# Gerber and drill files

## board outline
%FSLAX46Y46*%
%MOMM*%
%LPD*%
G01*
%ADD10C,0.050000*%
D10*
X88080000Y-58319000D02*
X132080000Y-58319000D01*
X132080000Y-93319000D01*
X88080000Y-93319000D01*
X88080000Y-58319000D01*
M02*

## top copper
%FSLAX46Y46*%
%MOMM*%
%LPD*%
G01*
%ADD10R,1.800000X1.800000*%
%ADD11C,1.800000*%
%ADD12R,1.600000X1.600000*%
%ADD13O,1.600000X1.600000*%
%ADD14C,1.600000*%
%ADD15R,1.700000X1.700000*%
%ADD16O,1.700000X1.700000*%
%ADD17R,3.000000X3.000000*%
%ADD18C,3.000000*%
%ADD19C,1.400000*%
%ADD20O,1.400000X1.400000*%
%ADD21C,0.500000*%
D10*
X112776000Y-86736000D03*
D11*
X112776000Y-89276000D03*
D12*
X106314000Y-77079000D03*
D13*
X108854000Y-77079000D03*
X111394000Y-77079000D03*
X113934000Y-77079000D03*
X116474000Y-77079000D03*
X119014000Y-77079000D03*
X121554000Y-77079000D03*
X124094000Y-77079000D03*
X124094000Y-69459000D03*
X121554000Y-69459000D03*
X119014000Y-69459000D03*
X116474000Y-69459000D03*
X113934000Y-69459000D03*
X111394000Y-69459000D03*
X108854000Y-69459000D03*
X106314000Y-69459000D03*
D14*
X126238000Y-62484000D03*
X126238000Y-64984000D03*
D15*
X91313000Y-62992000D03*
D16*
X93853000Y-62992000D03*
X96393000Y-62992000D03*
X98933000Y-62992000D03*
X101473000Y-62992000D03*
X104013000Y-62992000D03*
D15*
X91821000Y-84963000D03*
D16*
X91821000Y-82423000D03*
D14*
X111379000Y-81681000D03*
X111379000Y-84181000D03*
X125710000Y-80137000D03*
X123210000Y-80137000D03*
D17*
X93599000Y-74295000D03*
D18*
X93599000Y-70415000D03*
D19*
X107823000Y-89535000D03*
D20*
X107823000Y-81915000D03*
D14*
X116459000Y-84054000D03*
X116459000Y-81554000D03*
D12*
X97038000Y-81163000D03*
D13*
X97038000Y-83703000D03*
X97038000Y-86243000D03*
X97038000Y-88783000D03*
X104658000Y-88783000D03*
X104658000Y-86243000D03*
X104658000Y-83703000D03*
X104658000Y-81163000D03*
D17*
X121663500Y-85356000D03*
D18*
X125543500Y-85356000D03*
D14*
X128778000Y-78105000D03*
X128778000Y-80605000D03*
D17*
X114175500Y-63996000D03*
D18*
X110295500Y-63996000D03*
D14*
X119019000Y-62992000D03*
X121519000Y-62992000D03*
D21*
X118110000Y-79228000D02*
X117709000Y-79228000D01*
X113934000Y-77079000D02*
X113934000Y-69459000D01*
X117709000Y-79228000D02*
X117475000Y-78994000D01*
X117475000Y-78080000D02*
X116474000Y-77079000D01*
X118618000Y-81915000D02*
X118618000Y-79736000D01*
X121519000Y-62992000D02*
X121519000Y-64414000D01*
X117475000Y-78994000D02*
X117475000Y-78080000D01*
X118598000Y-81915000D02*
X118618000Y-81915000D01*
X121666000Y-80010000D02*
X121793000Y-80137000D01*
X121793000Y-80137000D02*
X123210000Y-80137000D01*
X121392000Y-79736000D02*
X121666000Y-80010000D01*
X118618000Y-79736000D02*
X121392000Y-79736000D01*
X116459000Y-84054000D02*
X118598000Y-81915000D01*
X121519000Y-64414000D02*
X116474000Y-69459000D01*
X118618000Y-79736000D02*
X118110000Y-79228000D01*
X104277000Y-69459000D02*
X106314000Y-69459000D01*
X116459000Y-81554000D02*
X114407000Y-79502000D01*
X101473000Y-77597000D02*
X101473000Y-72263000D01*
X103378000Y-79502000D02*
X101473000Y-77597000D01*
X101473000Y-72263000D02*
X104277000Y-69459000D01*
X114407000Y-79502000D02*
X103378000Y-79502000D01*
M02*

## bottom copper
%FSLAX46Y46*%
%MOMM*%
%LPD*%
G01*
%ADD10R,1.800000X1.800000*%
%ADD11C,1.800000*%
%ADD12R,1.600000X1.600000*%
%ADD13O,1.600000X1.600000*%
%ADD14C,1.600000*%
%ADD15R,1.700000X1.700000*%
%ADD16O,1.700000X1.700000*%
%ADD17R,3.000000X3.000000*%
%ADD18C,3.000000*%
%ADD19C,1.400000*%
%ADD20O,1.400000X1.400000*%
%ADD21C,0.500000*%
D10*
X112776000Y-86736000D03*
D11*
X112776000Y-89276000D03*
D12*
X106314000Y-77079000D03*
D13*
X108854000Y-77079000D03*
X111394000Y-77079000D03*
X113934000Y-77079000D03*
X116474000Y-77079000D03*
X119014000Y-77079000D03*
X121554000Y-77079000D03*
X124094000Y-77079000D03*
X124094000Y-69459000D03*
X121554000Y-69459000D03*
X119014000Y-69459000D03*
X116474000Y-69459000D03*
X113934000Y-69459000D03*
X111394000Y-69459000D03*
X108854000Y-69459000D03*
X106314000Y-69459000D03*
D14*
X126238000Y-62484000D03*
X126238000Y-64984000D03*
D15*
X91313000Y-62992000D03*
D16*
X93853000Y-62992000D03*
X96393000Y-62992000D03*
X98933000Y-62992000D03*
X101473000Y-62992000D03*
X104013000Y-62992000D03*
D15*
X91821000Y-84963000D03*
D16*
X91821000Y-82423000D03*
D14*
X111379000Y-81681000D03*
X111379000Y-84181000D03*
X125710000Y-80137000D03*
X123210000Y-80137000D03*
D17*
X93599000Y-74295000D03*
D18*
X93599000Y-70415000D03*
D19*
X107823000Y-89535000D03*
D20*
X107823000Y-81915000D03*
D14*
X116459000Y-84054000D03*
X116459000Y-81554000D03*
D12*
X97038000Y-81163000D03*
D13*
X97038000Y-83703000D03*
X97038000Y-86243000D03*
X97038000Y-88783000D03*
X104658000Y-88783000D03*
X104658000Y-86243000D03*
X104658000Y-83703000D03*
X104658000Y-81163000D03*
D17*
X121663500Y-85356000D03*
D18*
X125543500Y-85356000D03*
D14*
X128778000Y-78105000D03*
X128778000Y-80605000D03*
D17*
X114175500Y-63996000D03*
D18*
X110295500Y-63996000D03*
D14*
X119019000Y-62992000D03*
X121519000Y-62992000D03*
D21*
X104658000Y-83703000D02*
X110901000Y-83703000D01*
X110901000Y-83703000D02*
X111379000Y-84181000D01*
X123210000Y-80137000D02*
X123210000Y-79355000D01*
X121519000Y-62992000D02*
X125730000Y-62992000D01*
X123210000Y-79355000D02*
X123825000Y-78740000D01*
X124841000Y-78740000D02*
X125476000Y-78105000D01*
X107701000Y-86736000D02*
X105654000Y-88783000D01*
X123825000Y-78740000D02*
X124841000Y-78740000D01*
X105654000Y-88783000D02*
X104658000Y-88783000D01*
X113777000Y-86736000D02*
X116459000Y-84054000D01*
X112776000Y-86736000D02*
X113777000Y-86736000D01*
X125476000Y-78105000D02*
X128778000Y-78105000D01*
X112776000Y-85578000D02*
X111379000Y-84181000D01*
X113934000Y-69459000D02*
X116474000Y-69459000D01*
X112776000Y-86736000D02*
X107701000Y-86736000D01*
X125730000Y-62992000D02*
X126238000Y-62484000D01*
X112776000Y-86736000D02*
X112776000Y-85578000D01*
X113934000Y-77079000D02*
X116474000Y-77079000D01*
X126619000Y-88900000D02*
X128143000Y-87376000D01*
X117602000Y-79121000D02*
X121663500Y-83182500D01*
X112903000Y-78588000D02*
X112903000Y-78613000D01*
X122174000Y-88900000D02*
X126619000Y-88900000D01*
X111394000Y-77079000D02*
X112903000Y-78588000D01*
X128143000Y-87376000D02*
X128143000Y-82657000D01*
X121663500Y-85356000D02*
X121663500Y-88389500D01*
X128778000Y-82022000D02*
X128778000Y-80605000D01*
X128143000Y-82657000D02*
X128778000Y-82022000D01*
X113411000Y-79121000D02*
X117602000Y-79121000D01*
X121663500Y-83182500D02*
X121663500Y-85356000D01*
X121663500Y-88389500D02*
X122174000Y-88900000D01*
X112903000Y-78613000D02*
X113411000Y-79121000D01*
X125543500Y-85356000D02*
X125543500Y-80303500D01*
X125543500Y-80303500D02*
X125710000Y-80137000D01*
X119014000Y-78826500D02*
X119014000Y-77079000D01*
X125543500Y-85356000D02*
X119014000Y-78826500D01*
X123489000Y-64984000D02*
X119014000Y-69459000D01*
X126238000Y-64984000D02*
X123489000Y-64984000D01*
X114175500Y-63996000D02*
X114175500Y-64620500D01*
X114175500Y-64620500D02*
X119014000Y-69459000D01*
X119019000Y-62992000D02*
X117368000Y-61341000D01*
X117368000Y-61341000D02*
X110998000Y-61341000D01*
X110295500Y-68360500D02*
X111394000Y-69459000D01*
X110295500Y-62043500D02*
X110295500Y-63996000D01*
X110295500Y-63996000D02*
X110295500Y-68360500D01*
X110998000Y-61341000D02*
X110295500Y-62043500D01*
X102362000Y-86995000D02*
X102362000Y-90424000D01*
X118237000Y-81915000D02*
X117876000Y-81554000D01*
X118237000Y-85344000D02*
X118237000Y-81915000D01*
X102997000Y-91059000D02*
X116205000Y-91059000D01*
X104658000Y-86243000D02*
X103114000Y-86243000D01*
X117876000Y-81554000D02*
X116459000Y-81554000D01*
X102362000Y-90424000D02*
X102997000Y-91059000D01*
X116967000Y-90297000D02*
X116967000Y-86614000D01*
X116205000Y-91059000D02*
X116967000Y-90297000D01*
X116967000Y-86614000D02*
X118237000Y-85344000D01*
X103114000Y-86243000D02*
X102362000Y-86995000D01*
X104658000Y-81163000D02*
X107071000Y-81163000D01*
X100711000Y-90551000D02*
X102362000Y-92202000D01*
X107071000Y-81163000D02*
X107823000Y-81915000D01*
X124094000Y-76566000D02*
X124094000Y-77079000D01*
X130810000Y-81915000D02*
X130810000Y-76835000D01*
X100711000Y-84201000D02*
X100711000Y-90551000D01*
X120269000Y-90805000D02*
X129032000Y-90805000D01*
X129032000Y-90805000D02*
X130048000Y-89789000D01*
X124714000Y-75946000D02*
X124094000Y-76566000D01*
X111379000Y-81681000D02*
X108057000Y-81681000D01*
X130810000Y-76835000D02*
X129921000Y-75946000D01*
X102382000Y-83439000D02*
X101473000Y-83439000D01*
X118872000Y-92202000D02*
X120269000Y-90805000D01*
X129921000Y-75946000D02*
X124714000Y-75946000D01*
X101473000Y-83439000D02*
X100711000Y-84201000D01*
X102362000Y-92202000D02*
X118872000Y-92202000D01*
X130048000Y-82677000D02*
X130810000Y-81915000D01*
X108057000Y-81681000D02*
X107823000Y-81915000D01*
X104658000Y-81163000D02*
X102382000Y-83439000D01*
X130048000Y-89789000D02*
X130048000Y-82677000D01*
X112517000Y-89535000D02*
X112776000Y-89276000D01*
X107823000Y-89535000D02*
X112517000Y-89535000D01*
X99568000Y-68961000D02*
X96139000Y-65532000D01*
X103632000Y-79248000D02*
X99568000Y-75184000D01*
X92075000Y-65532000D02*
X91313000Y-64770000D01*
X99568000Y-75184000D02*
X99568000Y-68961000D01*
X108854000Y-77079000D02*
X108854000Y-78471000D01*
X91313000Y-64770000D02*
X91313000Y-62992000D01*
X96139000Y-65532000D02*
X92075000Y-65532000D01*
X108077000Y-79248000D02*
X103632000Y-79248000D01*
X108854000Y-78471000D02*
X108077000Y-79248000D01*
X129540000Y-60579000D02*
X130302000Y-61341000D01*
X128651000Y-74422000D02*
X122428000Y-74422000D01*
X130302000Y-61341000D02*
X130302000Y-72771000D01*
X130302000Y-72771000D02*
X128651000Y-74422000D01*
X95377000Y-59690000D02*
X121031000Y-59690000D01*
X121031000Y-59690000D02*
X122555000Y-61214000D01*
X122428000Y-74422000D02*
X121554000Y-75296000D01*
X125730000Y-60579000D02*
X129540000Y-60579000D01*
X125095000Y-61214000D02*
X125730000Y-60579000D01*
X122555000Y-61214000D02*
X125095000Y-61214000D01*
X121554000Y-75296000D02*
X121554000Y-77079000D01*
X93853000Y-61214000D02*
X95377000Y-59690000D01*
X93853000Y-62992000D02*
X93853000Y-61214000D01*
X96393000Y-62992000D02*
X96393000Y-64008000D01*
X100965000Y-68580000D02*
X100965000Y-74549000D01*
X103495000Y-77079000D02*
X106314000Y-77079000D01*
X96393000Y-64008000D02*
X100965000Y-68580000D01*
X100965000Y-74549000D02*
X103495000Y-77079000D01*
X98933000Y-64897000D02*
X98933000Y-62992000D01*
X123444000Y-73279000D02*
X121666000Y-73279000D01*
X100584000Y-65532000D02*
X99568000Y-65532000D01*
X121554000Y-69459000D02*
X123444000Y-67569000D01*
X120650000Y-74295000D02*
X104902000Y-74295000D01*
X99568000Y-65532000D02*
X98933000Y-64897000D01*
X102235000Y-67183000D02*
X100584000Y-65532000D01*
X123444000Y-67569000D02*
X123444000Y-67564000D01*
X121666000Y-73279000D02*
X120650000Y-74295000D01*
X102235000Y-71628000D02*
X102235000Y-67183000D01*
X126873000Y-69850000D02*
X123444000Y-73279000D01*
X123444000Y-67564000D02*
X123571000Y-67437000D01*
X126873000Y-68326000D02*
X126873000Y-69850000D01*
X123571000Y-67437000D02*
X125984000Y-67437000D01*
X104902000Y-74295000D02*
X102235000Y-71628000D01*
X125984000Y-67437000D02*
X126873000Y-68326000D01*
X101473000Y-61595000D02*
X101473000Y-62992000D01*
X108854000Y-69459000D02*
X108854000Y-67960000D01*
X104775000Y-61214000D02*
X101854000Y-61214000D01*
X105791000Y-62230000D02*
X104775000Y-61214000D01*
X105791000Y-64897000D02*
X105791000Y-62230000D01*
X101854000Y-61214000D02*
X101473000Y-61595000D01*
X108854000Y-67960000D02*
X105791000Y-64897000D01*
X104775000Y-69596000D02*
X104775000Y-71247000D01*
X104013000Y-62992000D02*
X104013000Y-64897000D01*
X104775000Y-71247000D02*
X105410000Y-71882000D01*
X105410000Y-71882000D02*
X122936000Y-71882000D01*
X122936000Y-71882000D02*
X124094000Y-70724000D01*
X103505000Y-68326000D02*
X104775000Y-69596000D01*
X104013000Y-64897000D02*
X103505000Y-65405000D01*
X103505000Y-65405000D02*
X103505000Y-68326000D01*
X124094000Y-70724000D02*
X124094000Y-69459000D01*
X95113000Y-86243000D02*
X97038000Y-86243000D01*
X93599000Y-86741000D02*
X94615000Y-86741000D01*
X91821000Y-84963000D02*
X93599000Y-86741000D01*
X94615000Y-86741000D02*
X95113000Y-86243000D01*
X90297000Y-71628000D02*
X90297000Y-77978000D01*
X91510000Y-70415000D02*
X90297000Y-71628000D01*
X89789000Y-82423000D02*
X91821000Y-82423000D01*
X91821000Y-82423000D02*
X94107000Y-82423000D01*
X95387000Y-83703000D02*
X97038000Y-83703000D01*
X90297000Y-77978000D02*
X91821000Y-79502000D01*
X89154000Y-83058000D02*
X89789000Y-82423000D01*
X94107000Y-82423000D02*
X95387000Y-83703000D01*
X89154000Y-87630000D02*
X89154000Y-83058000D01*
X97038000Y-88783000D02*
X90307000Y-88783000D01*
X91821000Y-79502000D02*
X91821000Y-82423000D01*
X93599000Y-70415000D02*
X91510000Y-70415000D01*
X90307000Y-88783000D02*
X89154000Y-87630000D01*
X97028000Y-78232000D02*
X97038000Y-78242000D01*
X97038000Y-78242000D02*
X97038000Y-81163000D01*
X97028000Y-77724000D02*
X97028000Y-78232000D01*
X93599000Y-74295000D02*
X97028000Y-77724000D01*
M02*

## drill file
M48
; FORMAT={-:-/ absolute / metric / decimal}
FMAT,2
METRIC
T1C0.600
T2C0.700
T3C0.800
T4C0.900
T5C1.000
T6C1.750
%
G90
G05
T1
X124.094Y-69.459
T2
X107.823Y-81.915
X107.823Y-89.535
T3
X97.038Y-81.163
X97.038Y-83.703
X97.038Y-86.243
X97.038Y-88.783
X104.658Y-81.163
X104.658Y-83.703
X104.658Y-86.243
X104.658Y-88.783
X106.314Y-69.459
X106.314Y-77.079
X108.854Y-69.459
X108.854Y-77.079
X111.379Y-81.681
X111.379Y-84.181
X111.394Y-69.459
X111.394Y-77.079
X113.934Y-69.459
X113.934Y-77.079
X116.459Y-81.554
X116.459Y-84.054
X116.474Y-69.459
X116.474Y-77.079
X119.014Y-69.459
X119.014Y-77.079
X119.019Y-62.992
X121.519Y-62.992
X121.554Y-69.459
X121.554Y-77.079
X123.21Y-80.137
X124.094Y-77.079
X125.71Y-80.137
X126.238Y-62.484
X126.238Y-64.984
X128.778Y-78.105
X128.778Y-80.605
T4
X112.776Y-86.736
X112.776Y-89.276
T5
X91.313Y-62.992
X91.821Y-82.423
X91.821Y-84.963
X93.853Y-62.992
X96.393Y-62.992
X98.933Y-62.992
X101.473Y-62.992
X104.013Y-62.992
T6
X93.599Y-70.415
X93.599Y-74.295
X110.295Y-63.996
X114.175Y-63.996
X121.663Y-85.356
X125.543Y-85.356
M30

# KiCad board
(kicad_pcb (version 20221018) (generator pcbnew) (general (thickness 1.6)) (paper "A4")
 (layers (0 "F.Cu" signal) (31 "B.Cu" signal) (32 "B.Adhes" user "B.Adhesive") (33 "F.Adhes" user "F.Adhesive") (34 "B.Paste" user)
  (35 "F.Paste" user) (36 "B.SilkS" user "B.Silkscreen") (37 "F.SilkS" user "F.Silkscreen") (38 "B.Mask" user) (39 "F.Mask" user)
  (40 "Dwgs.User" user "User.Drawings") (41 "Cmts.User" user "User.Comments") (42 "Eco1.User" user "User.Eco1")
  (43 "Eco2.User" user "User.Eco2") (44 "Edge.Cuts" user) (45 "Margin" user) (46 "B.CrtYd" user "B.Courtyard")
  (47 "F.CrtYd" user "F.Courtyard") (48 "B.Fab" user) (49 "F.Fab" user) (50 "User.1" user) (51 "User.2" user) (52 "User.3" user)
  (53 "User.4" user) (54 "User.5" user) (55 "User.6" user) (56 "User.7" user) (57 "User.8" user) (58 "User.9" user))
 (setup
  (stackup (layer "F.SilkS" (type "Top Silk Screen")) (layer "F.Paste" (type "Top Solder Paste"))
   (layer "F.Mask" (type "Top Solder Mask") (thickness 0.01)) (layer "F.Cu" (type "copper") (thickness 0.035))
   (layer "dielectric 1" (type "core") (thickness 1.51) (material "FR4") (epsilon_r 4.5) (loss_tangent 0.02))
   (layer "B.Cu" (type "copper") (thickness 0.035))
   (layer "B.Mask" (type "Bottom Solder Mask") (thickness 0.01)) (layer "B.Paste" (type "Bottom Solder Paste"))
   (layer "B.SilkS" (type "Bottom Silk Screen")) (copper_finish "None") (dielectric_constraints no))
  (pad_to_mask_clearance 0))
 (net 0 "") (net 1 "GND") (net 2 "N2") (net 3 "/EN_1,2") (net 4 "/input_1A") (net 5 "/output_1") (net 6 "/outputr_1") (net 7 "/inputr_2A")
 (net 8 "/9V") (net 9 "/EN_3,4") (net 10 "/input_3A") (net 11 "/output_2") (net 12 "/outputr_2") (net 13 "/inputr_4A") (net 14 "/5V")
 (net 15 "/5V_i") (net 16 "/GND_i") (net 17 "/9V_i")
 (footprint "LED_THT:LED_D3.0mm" (layer "F.Cu") (at 112.776 86.736 -90)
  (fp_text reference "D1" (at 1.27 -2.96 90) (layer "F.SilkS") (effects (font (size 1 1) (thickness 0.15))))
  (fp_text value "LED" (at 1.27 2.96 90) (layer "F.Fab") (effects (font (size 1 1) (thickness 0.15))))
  (pad "1" thru_hole rect (at 0 0 270) (size 1.8 1.8) (drill 0.9) (layers "*.Cu" "*.Mask") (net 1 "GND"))
  (pad "2" thru_hole circle (at 2.54 0 270) (size 1.8 1.8) (drill 0.9) (layers "*.Cu" "*.Mask") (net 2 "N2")))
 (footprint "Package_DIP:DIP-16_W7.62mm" (layer "F.Cu") (at 106.314 77.079 90)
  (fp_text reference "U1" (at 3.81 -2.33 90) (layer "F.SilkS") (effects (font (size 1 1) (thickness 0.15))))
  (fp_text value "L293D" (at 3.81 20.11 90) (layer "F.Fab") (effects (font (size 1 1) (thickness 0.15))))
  (pad "1" thru_hole rect (at 0 0 90) (size 1.6 1.6) (drill 0.8) (layers "*.Cu" "*.Mask") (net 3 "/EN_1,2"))
  (pad "2" thru_hole oval (at 0 2.54 90) (size 1.6 1.6) (drill 0.8) (layers "*.Cu" "*.Mask") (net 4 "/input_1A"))
  (pad "3" thru_hole oval (at 0 5.08 90) (size 1.6 1.6) (drill 0.8) (layers "*.Cu" "*.Mask") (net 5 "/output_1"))
  (pad "4" thru_hole oval (at 0 7.62 90) (size 1.6 1.6) (drill 0.8) (layers "*.Cu" "*.Mask") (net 1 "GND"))
  (pad "5" thru_hole oval (at 0 10.16 90) (size 1.6 1.6) (drill 0.8) (layers "*.Cu" "*.Mask") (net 1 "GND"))
  (pad "6" thru_hole oval (at 0 12.7 90) (size 1.6 1.6) (drill 0.8) (layers "*.Cu" "*.Mask") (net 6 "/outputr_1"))
  (pad "7" thru_hole oval (at 0 15.24 90) (size 1.6 1.6) (drill 0.8) (layers "*.Cu" "*.Mask") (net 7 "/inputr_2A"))
  (pad "8" thru_hole oval (at 0 17.78 90) (size 1.6 1.6) (drill 0.8) (layers "*.Cu" "*.Mask") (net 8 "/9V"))
  (pad "9" thru_hole oval (at 7.62 17.78 90) (size 1.6 1.6) (drill 0.6) (layers "*.Cu" "*.Mask") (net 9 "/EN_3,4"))
  (pad "10" thru_hole oval (at 7.62 15.24 90) (size 1.6 1.6) (drill 0.8) (layers "*.Cu" "*.Mask") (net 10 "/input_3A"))
  (pad "11" thru_hole oval (at 7.62 12.7 90) (size 1.6 1.6) (drill 0.8) (layers "*.Cu" "*.Mask") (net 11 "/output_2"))
  (pad "12" thru_hole oval (at 7.62 10.16 90) (size 1.6 1.6) (drill 0.8) (layers "*.Cu" "*.Mask") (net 1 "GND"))
  (pad "13" thru_hole oval (at 7.62 7.62 90) (size 1.6 1.6) (drill 0.8) (layers "*.Cu" "*.Mask") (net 1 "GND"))
  (pad "14" thru_hole oval (at 7.62 5.08 90) (size 1.6 1.6) (drill 0.8) (layers "*.Cu" "*.Mask") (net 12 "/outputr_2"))
  (pad "15" thru_hole oval (at 7.62 2.54 90) (size 1.6 1.6) (drill 0.8) (layers "*.Cu" "*.Mask") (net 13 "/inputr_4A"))
  (pad "16" thru_hole oval (at 7.62 0 90) (size 1.6 1.6) (drill 0.8) (layers "*.Cu" "*.Mask") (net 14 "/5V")))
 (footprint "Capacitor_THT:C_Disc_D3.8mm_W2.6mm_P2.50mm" (layer "F.Cu") (at 126.238 62.484 -90)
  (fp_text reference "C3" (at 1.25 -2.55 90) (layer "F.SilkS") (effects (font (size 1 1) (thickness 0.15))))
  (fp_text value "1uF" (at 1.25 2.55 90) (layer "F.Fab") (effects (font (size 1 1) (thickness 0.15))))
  (pad "1" thru_hole circle (at 0 0 270) (size 1.6 1.6) (drill 0.8) (layers "*.Cu" "*.Mask") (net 1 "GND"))
  (pad "2" thru_hole circle (at 2.5 0 270) (size 1.6 1.6) (drill 0.8) (layers "*.Cu" "*.Mask") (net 11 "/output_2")))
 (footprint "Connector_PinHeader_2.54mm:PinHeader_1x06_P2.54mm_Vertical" (layer "F.Cu") (at 91.313 62.992 90)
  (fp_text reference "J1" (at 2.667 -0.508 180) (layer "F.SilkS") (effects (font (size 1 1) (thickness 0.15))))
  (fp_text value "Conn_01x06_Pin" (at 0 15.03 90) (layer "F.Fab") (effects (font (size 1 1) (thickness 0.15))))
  (pad "1" thru_hole rect (at 0 0 90) (size 1.7 1.7) (drill 1) (layers "*.Cu" "*.Mask") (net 4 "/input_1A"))
  (pad "2" thru_hole oval (at 0 2.54 90) (size 1.7 1.7) (drill 1) (layers "*.Cu" "*.Mask") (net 7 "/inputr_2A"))
  (pad "3" thru_hole oval (at 0 5.08 90) (size 1.7 1.7) (drill 1) (layers "*.Cu" "*.Mask") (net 3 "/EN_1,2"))
  (pad "4" thru_hole oval (at 0 7.62 90) (size 1.7 1.7) (drill 1) (layers "*.Cu" "*.Mask") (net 10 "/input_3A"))
  (pad "5" thru_hole oval (at 0 10.16 90) (size 1.7 1.7) (drill 1) (layers "*.Cu" "*.Mask") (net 13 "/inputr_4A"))
  (pad "6" thru_hole oval (at 0 12.7 90) (size 1.7 1.7) (drill 1) (layers "*.Cu" "*.Mask") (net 9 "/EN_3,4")))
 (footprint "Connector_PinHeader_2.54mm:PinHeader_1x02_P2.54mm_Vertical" (layer "F.Cu") (at 91.821 84.963 180)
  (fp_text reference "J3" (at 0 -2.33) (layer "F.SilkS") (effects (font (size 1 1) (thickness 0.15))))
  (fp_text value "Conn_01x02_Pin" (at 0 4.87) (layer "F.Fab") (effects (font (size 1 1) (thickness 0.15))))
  (pad "1" thru_hole rect (at 0 0 180) (size 1.7 1.7) (drill 1) (layers "*.Cu" "*.Mask") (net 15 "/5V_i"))
  (pad "2" thru_hole oval (at 0 2.54 180) (size 1.7 1.7) (drill 1) (layers "*.Cu" "*.Mask") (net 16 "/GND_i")))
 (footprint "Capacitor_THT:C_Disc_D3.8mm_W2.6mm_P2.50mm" (layer "F.Cu") (at 111.379 81.681 -90)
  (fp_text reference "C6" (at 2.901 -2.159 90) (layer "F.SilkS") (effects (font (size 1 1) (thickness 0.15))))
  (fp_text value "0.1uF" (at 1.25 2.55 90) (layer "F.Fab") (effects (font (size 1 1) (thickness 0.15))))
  (pad "1" thru_hole circle (at 0 0 270) (size 1.6 1.6) (drill 0.8) (layers "*.Cu" "*.Mask") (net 8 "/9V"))
  (pad "2" thru_hole circle (at 2.5 0 270) (size 1.6 1.6) (drill 0.8) (layers "*.Cu" "*.Mask") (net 1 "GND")))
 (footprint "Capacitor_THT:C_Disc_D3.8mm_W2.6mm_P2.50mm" (layer "F.Cu") (at 125.71 80.137 180)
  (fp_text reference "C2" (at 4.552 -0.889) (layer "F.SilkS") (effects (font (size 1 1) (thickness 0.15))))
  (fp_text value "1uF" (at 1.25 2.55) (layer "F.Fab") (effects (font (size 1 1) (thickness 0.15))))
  (pad "1" thru_hole circle (at 0 0 180) (size 1.6 1.6) (drill 0.8) (layers "*.Cu" "*.Mask") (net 6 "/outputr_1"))
  (pad "2" thru_hole circle (at 2.5 0 180) (size 1.6 1.6) (drill 0.8) (layers "*.Cu" "*.Mask") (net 1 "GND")))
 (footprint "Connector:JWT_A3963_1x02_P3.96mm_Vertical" (layer "F.Cu") (at 93.599 74.295 90)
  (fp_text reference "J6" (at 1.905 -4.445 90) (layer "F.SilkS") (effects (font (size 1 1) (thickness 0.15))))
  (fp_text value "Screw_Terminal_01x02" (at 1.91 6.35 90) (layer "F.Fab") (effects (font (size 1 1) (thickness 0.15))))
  (pad "1" thru_hole rect (at 0 0 90) (size 3 3) (drill 1.75) (layers "*.Cu" "*.Mask") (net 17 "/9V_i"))
  (pad "2" thru_hole circle (at 3.88 0 90) (size 3 3) (drill 1.75) (layers "*.Cu" "*.Mask") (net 16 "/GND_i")))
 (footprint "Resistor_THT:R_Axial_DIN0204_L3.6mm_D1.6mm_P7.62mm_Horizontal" (layer "F.Cu") (at 107.823 89.535 90)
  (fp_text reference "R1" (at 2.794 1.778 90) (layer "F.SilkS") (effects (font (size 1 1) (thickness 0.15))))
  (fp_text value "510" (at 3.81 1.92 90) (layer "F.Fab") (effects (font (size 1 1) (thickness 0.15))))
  (pad "1" thru_hole circle (at 0 0 90) (size 1.4 1.4) (drill 0.7) (layers "*.Cu" "*.Mask") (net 2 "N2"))
  (pad "2" thru_hole oval (at 7.62 0 90) (size 1.4 1.4) (drill 0.7) (layers "*.Cu" "*.Mask") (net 8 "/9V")))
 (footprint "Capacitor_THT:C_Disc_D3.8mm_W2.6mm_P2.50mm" (layer "F.Cu") (at 116.459 84.054 90)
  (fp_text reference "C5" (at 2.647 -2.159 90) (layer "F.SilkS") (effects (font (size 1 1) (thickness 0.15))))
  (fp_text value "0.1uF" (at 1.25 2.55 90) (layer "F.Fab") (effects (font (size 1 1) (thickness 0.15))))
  (pad "1" thru_hole circle (at 0 0 90) (size 1.6 1.6) (drill 0.8) (layers "*.Cu" "*.Mask") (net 1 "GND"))
  (pad "2" thru_hole circle (at 2.5 0 90) (size 1.6 1.6) (drill 0.8) (layers "*.Cu" "*.Mask") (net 14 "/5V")))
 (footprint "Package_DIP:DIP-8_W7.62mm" (layer "F.Cu") (at 97.038 81.163)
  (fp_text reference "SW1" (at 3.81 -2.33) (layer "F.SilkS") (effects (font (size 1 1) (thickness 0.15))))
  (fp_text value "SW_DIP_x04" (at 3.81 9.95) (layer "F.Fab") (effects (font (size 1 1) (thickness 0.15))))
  (pad "1" thru_hole rect (at 0 0) (size 1.6 1.6) (drill 0.8) (layers "*.Cu" "*.Mask") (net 17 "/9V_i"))
  (pad "2" thru_hole oval (at 0 2.54) (size 1.6 1.6) (drill 0.8) (layers "*.Cu" "*.Mask") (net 16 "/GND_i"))
  (pad "3" thru_hole oval (at 0 5.08) (size 1.6 1.6) (drill 0.8) (layers "*.Cu" "*.Mask") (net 15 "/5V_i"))
  (pad "4" thru_hole oval (at 0 7.62) (size 1.6 1.6) (drill 0.8) (layers "*.Cu" "*.Mask") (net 16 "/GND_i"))
  (pad "5" thru_hole oval (at 7.62 7.62) (size 1.6 1.6) (drill 0.8) (layers "*.Cu" "*.Mask") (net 1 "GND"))
  (pad "6" thru_hole oval (at 7.62 5.08) (size 1.6 1.6) (drill 0.8) (layers "*.Cu" "*.Mask") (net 14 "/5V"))
  (pad "7" thru_hole oval (at 7.62 2.54) (size 1.6 1.6) (drill 0.8) (layers "*.Cu" "*.Mask") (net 1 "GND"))
  (pad "8" thru_hole oval (at 7.62 0) (size 1.6 1.6) (drill 0.8) (layers "*.Cu" "*.Mask") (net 8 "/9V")))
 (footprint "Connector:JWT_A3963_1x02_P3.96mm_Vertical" (layer "F.Cu") (at 121.6635 85.356)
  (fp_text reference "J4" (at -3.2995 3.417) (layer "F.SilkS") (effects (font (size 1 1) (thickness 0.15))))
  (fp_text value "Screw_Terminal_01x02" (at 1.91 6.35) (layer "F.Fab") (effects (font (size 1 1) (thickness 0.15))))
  (pad "1" thru_hole rect (at 0 0) (size 3 3) (drill 1.75) (layers "*.Cu" "*.Mask") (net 5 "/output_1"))
  (pad "2" thru_hole circle (at 3.88 0) (size 3 3) (drill 1.75) (layers "*.Cu" "*.Mask") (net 6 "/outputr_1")))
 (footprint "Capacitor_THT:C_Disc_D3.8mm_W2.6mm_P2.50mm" (layer "F.Cu") (at 128.778 78.105 -90)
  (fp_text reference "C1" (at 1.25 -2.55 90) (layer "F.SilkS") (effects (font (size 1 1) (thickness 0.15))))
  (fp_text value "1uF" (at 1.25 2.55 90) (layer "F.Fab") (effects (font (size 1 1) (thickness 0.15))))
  (pad "1" thru_hole circle (at 0 0 270) (size 1.6 1.6) (drill 0.8) (layers "*.Cu" "*.Mask") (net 1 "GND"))
  (pad "2" thru_hole circle (at 2.5 0 270) (size 1.6 1.6) (drill 0.8) (layers "*.Cu" "*.Mask") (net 5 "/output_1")))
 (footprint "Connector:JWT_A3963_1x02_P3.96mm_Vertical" (layer "F.Cu") (at 114.1755 63.996 180)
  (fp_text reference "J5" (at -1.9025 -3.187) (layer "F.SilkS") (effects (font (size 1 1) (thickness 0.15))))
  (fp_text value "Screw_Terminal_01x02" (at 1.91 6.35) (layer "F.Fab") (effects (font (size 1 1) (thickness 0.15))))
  (pad "1" thru_hole rect (at 0 0 180) (size 3 3) (drill 1.75) (layers "*.Cu" "*.Mask") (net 11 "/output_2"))
  (pad "2" thru_hole circle (at 3.88 0 180) (size 3 3) (drill 1.75) (layers "*.Cu" "*.Mask") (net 12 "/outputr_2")))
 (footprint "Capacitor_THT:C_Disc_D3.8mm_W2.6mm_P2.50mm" (layer "F.Cu") (at 119.019 62.992)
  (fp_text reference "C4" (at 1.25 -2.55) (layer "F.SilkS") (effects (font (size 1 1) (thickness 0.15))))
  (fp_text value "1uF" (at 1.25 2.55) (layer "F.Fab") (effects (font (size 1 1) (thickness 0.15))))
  (pad "1" thru_hole circle (at 0 0) (size 1.6 1.6) (drill 0.8) (layers "*.Cu" "*.Mask") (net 12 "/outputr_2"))
  (pad "2" thru_hole circle (at 2.5 0) (size 1.6 1.6) (drill 0.8) (layers "*.Cu" "*.Mask") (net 1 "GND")))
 (gr_rect (start 88.08 58.319) (end 132.08 93.319) (stroke (width 0.05) (type default)) (fill none) (layer "Edge.Cuts"))
 (segment (start 118.11 79.228) (end 117.709 79.228) (width 0.5) (layer "F.Cu") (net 1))
 (segment (start 113.934 77.079) (end 113.934 69.459) (width 0.5) (layer "F.Cu") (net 1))
 (segment (start 117.709 79.228) (end 117.475 78.994) (width 0.5) (layer "F.Cu") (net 1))
 (segment (start 117.475 78.08) (end 116.474 77.079) (width 0.5) (layer "F.Cu") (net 1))
 (segment (start 118.618 81.915) (end 118.618 79.736) (width 0.5) (layer "F.Cu") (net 1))
 (segment (start 121.519 62.992) (end 121.519 64.414) (width 0.5) (layer "F.Cu") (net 1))
 (segment (start 117.475 78.994) (end 117.475 78.08) (width 0.5) (layer "F.Cu") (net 1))
 (segment (start 118.598 81.915) (end 118.618 81.915) (width 0.5) (layer "F.Cu") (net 1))
 (segment (start 121.666 80.01) (end 121.793 80.137) (width 0.5) (layer "F.Cu") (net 1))
 (segment (start 121.793 80.137) (end 123.21 80.137) (width 0.5) (layer "F.Cu") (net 1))
 (segment (start 121.392 79.736) (end 121.666 80.01) (width 0.5) (layer "F.Cu") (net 1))
 (segment (start 118.618 79.736) (end 121.392 79.736) (width 0.5) (layer "F.Cu") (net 1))
 (segment (start 116.459 84.054) (end 118.598 81.915) (width 0.5) (layer "F.Cu") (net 1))
 (segment (start 121.519 64.414) (end 116.474 69.459) (width 0.5) (layer "F.Cu") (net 1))
 (segment (start 118.618 79.736) (end 118.11 79.228) (width 0.5) (layer "F.Cu") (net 1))
 (segment (start 104.658 83.703) (end 110.901 83.703) (width 0.5) (layer "B.Cu") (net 1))
 (segment (start 110.901 83.703) (end 111.379 84.181) (width 0.5) (layer "B.Cu") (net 1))
 (segment (start 123.21 80.137) (end 123.21 79.355) (width 0.5) (layer "B.Cu") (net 1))
 (segment (start 121.519 62.992) (end 125.73 62.992) (width 0.5) (layer "B.Cu") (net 1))
 (segment (start 123.21 79.355) (end 123.825 78.74) (width 0.5) (layer "B.Cu") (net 1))
 (segment (start 124.841 78.74) (end 125.476 78.105) (width 0.5) (layer "B.Cu") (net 1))
 (segment (start 107.701 86.736) (end 105.654 88.783) (width 0.5) (layer "B.Cu") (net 1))
 (segment (start 123.825 78.74) (end 124.841 78.74) (width 0.5) (layer "B.Cu") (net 1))
 (segment (start 105.654 88.783) (end 104.658 88.783) (width 0.5) (layer "B.Cu") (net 1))
 (segment (start 113.777 86.736) (end 116.459 84.054) (width 0.5) (layer "B.Cu") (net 1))
 (segment (start 112.776 86.736) (end 113.777 86.736) (width 0.5) (layer "B.Cu") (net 1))
 (segment (start 125.476 78.105) (end 128.778 78.105) (width 0.5) (layer "B.Cu") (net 1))
 (segment (start 112.776 85.578) (end 111.379 84.181) (width 0.5) (layer "B.Cu") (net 1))
 (segment (start 113.934 69.459) (end 116.474 69.459) (width 0.5) (layer "B.Cu") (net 1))
 (segment (start 112.776 86.736) (end 107.701 86.736) (width 0.5) (layer "B.Cu") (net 1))
 (segment (start 125.73 62.992) (end 126.238 62.484) (width 0.5) (layer "B.Cu") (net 1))
 (segment (start 112.776 86.736) (end 112.776 85.578) (width 0.5) (layer "B.Cu") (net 1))
 (segment (start 113.934 77.079) (end 116.474 77.079) (width 0.5) (layer "B.Cu") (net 1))
 (segment (start 126.619 88.9) (end 128.143 87.376) (width 0.5) (layer "B.Cu") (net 5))
 (segment (start 117.602 79.121) (end 121.6635 83.1825) (width 0.5) (layer "B.Cu") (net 5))
 (segment (start 112.903 78.588) (end 112.903 78.613) (width 0.5) (layer "B.Cu") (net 5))
 (segment (start 122.174 88.9) (end 126.619 88.9) (width 0.5) (layer "B.Cu") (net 5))
 (segment (start 111.394 77.079) (end 112.903 78.588) (width 0.5) (layer "B.Cu") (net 5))
 (segment (start 128.143 87.376) (end 128.143 82.657) (width 0.5) (layer "B.Cu") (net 5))
 (segment (start 121.6635 85.356) (end 121.6635 88.3895) (width 0.5) (layer "B.Cu") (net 5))
 (segment (start 128.778 82.022) (end 128.778 80.605) (width 0.5) (layer "B.Cu") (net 5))
 (segment (start 128.143 82.657) (end 128.778 82.022) (width 0.5) (layer "B.Cu") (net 5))
 (segment (start 113.411 79.121) (end 117.602 79.121) (width 0.5) (layer "B.Cu") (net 5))
 (segment (start 121.6635 83.1825) (end 121.6635 85.356) (width 0.5) (layer "B.Cu") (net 5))
 (segment (start 121.6635 88.3895) (end 122.174 88.9) (width 0.5) (layer "B.Cu") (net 5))
 (segment (start 112.903 78.613) (end 113.411 79.121) (width 0.5) (layer "B.Cu") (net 5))
 (segment (start 125.5435 85.356) (end 125.5435 80.3035) (width 0.5) (layer "B.Cu") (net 6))
 (segment (start 125.5435 80.3035) (end 125.71 80.137) (width 0.5) (layer "B.Cu") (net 6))
 (segment (start 119.014 78.8265) (end 119.014 77.079) (width 0.5) (layer "B.Cu") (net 6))
 (segment (start 125.5435 85.356) (end 119.014 78.8265) (width 0.5) (layer "B.Cu") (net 6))
 (segment (start 123.489 64.984) (end 119.014 69.459) (width 0.5) (layer "B.Cu") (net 11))
 (segment (start 126.238 64.984) (end 123.489 64.984) (width 0.5) (layer "B.Cu") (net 11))
 (segment (start 114.1755 63.996) (end 114.1755 64.6205) (width 0.5) (layer "B.Cu") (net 11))
 (segment (start 114.1755 64.6205) (end 119.014 69.459) (width 0.5) (layer "B.Cu") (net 11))
 (segment (start 119.019 62.992) (end 117.368 61.341) (width 0.5) (layer "B.Cu") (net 12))
 (segment (start 117.368 61.341) (end 110.998 61.341) (width 0.5) (layer "B.Cu") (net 12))
 (segment (start 110.2955 68.3605) (end 111.394 69.459) (width 0.5) (layer "B.Cu") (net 12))
 (segment (start 110.2955 62.0435) (end 110.2955 63.996) (width 0.5) (layer "B.Cu") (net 12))
 (segment (start 110.2955 63.996) (end 110.2955 68.3605) (width 0.5) (layer "B.Cu") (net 12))
 (segment (start 110.998 61.341) (end 110.2955 62.0435) (width 0.5) (layer "B.Cu") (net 12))
 (segment (start 104.277 69.459) (end 106.314 69.459) (width 0.5) (layer "F.Cu") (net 14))
 (segment (start 116.459 81.554) (end 114.407 79.502) (width 0.5) (layer "F.Cu") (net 14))
 (segment (start 101.473 77.597) (end 101.473 72.263) (width 0.5) (layer "F.Cu") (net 14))
 (segment (start 103.378 79.502) (end 101.473 77.597) (width 0.5) (layer "F.Cu") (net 14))
 (segment (start 101.473 72.263) (end 104.277 69.459) (width 0.5) (layer "F.Cu") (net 14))
 (segment (start 114.407 79.502) (end 103.378 79.502) (width 0.5) (layer "F.Cu") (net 14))
 (segment (start 102.362 86.995) (end 102.362 90.424) (width 0.5) (layer "B.Cu") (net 14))
 (segment (start 118.237 81.915) (end 117.876 81.554) (width 0.5) (layer "B.Cu") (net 14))
 (segment (start 118.237 85.344) (end 118.237 81.915) (width 0.5) (layer "B.Cu") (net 14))
 (segment (start 102.997 91.059) (end 116.205 91.059) (width 0.5) (layer "B.Cu") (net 14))
 (segment (start 104.658 86.243) (end 103.114 86.243) (width 0.5) (layer "B.Cu") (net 14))
 (segment (start 117.876 81.554) (end 116.459 81.554) (width 0.5) (layer "B.Cu") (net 14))
 (segment (start 102.362 90.424) (end 102.997 91.059) (width 0.5) (layer "B.Cu") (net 14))
 (segment (start 116.967 90.297) (end 116.967 86.614) (width 0.5) (layer "B.Cu") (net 14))
 (segment (start 116.205 91.059) (end 116.967 90.297) (width 0.5) (layer "B.Cu") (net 14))
 (segment (start 116.967 86.614) (end 118.237 85.344) (width 0.5) (layer "B.Cu") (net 14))
 (segment (start 103.114 86.243) (end 102.362 86.995) (width 0.5) (layer "B.Cu") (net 14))
 (segment (start 104.658 81.163) (end 107.071 81.163) (width 0.5) (layer "B.Cu") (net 8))
 (segment (start 100.711 90.551) (end 102.362 92.202) (width 0.5) (layer "B.Cu") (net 8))
 (segment (start 107.071 81.163) (end 107.823 81.915) (width 0.5) (layer "B.Cu") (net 8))
 (segment (start 124.094 76.566) (end 124.094 77.079) (width 0.5) (layer "B.Cu") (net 8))
 (segment (start 130.81 81.915) (end 130.81 76.835) (width 0.5) (layer "B.Cu") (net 8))
 (segment (start 100.711 84.201) (end 100.711 90.551) (width 0.5) (layer "B.Cu") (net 8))
 (segment (start 120.269 90.805) (end 129.032 90.805) (width 0.5) (layer "B.Cu") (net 8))
 (segment (start 129.032 90.805) (end 130.048 89.789) (width 0.5) (layer "B.Cu") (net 8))
 (segment (start 124.714 75.946) (end 124.094 76.566) (width 0.5) (layer "B.Cu") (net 8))
 (segment (start 111.379 81.681) (end 108.057 81.681) (width 0.5) (layer "B.Cu") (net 8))
 (segment (start 130.81 76.835) (end 129.921 75.946) (width 0.5) (layer "B.Cu") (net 8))
 (segment (start 102.382 83.439) (end 101.473 83.439) (width 0.5) (layer "B.Cu") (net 8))
 (segment (start 118.872 92.202) (end 120.269 90.805) (width 0.5) (layer "B.Cu") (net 8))
 (segment (start 129.921 75.946) (end 124.714 75.946) (width 0.5) (layer "B.Cu") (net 8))
 (segment (start 101.473 83.439) (end 100.711 84.201) (width 0.5) (layer "B.Cu") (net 8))
 (segment (start 102.362 92.202) (end 118.872 92.202) (width 0.5) (layer "B.Cu") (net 8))
 (segment (start 130.048 82.677) (end 130.81 81.915) (width 0.5) (layer "B.Cu") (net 8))
 (segment (start 108.057 81.681) (end 107.823 81.915) (width 0.5) (layer "B.Cu") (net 8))
 (segment (start 104.658 81.163) (end 102.382 83.439) (width 0.5) (layer "B.Cu") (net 8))
 (segment (start 130.048 89.789) (end 130.048 82.677) (width 0.5) (layer "B.Cu") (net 8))
 (segment (start 112.517 89.535) (end 112.776 89.276) (width 0.5) (layer "B.Cu") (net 2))
 (segment (start 107.823 89.535) (end 112.517 89.535) (width 0.5) (layer "B.Cu") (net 2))
 (segment (start 99.568 68.961) (end 96.139 65.532) (width 0.5) (layer "B.Cu") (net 4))
 (segment (start 103.632 79.248) (end 99.568 75.184) (width 0.5) (layer "B.Cu") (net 4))
 (segment (start 92.075 65.532) (end 91.313 64.77) (width 0.5) (layer "B.Cu") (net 4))
 (segment (start 99.568 75.184) (end 99.568 68.961) (width 0.5) (layer "B.Cu") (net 4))
 (segment (start 108.854 77.079) (end 108.854 78.471) (width 0.5) (layer "B.Cu") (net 4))
 (segment (start 91.313 64.77) (end 91.313 62.992) (width 0.5) (layer "B.Cu") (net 4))
 (segment (start 96.139 65.532) (end 92.075 65.532) (width 0.5) (layer "B.Cu") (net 4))
 (segment (start 108.077 79.248) (end 103.632 79.248) (width 0.5) (layer "B.Cu") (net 4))
 (segment (start 108.854 78.471) (end 108.077 79.248) (width 0.5) (layer "B.Cu") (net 4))
 (segment (start 129.54 60.579) (end 130.302 61.341) (width 0.5) (layer "B.Cu") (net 7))
 (segment (start 128.651 74.422) (end 122.428 74.422) (width 0.5) (layer "B.Cu") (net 7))
 (segment (start 130.302 61.341) (end 130.302 72.771) (width 0.5) (layer "B.Cu") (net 7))
 (segment (start 130.302 72.771) (end 128.651 74.422) (width 0.5) (layer "B.Cu") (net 7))
 (segment (start 95.377 59.69) (end 121.031 59.69) (width 0.5) (layer "B.Cu") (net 7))
 (segment (start 121.031 59.69) (end 122.555 61.214) (width 0.5) (layer "B.Cu") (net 7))
 (segment (start 122.428 74.422) (end 121.554 75.296) (width 0.5) (layer "B.Cu") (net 7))
 (segment (start 125.73 60.579) (end 129.54 60.579) (width 0.5) (layer "B.Cu") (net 7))
 (segment (start 125.095 61.214) (end 125.73 60.579) (width 0.5) (layer "B.Cu") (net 7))
 (segment (start 122.555 61.214) (end 125.095 61.214) (width 0.5) (layer "B.Cu") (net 7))
 (segment (start 121.554 75.296) (end 121.554 77.079) (width 0.5) (layer "B.Cu") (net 7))
 (segment (start 93.853 61.214) (end 95.377 59.69) (width 0.5) (layer "B.Cu") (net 7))
 (segment (start 93.853 62.992) (end 93.853 61.214) (width 0.5) (layer "B.Cu") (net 7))
 (segment (start 96.393 62.992) (end 96.393 64.008) (width 0.5) (layer "B.Cu") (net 3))
 (segment (start 100.965 68.58) (end 100.965 74.549) (width 0.5) (layer "B.Cu") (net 3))
 (segment (start 103.495 77.079) (end 106.314 77.079) (width 0.5) (layer "B.Cu") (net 3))
 (segment (start 96.393 64.008) (end 100.965 68.58) (width 0.5) (layer "B.Cu") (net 3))
 (segment (start 100.965 74.549) (end 103.495 77.079) (width 0.5) (layer "B.Cu") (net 3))
 (segment (start 98.933 64.897) (end 98.933 62.992) (width 0.5) (layer "B.Cu") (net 10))
 (segment (start 123.444 73.279) (end 121.666 73.279) (width 0.5) (layer "B.Cu") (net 10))
 (segment (start 100.584 65.532) (end 99.568 65.532) (width 0.5) (layer "B.Cu") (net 10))
 (segment (start 121.554 69.459) (end 123.444 67.569) (width 0.5) (layer "B.Cu") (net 10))
 (segment (start 120.65 74.295) (end 104.902 74.295) (width 0.5) (layer "B.Cu") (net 10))
 (segment (start 99.568 65.532) (end 98.933 64.897) (width 0.5) (layer "B.Cu") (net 10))
 (segment (start 102.235 67.183) (end 100.584 65.532) (width 0.5) (layer "B.Cu") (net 10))
 (segment (start 123.444 67.569) (end 123.444 67.564) (width 0.5) (layer "B.Cu") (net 10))
 (segment (start 121.666 73.279) (end 120.65 74.295) (width 0.5) (layer "B.Cu") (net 10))
 (segment (start 102.235 71.628) (end 102.235 67.183) (width 0.5) (layer "B.Cu") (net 10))
 (segment (start 126.873 69.85) (end 123.444 73.279) (width 0.5) (layer "B.Cu") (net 10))
 (segment (start 123.444 67.564) (end 123.571 67.437) (width 0.5) (layer "B.Cu") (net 10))
 (segment (start 126.873 68.326) (end 126.873 69.85) (width 0.5) (layer "B.Cu") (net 10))
 (segment (start 123.571 67.437) (end 125.984 67.437) (width 0.5) (layer "B.Cu") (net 10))
 (segment (start 104.902 74.295) (end 102.235 71.628) (width 0.5) (layer "B.Cu") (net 10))
 (segment (start 125.984 67.437) (end 126.873 68.326) (width 0.5) (layer "B.Cu") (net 10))
 (segment (start 101.473 61.595) (end 101.473 62.992) (width 0.5) (layer "B.Cu") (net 13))
 (segment (start 108.854 69.459) (end 108.854 67.96) (width 0.5) (layer "B.Cu") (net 13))
 (segment (start 104.775 61.214) (end 101.854 61.214) (width 0.5) (layer "B.Cu") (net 13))
 (segment (start 105.791 62.23) (end 104.775 61.214) (width 0.5) (layer "B.Cu") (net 13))
 (segment (start 105.791 64.897) (end 105.791 62.23) (width 0.5) (layer "B.Cu") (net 13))
 (segment (start 101.854 61.214) (end 101.473 61.595) (width 0.5) (layer "B.Cu") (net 13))
 (segment (start 108.854 67.96) (end 105.791 64.897) (width 0.5) (layer "B.Cu") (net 13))
 (segment (start 104.775 69.596) (end 104.775 71.247) (width 0.5) (layer "B.Cu") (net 9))
 (segment (start 104.013 62.992) (end 104.013 64.897) (width 0.5) (layer "B.Cu") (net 9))
 (segment (start 104.775 71.247) (end 105.41 71.882) (width 0.5) (layer "B.Cu") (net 9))
 (segment (start 105.41 71.882) (end 122.936 71.882) (width 0.5) (layer "B.Cu") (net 9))
 (segment (start 122.936 71.882) (end 124.094 70.724) (width 0.5) (layer "B.Cu") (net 9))
 (segment (start 103.505 68.326) (end 104.775 69.596) (width 0.5) (layer "B.Cu") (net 9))
 (segment (start 104.013 64.897) (end 103.505 65.405) (width 0.5) (layer "B.Cu") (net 9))
 (segment (start 103.505 65.405) (end 103.505 68.326) (width 0.5) (layer "B.Cu") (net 9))
 (segment (start 124.094 70.724) (end 124.094 69.459) (width 0.5) (layer "B.Cu") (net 9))
 (segment (start 95.113 86.243) (end 97.038 86.243) (width 0.5) (layer "B.Cu") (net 15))
 (segment (start 93.599 86.741) (end 94.615 86.741) (width 0.5) (layer "B.Cu") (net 15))
 (segment (start 91.821 84.963) (end 93.599 86.741) (width 0.5) (layer "B.Cu") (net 15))
 (segment (start 94.615 86.741) (end 95.113 86.243) (width 0.5) (layer "B.Cu") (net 15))
 (segment (start 90.297 71.628) (end 90.297 77.978) (width 0.5) (layer "B.Cu") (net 16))
 (segment (start 91.51 70.415) (end 90.297 71.628) (width 0.5) (layer "B.Cu") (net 16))
 (segment (start 89.789 82.423) (end 91.821 82.423) (width 0.5) (layer "B.Cu") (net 16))
 (segment (start 91.821 82.423) (end 94.107 82.423) (width 0.5) (layer "B.Cu") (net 16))
 (segment (start 95.387 83.703) (end 97.038 83.703) (width 0.5) (layer "B.Cu") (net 16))
 (segment (start 90.297 77.978) (end 91.821 79.502) (width 0.5) (layer "B.Cu") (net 16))
 (segment (start 89.154 83.058) (end 89.789 82.423) (width 0.5) (layer "B.Cu") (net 16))
 (segment (start 94.107 82.423) (end 95.387 83.703) (width 0.5) (layer "B.Cu") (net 16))
 (segment (start 89.154 87.63) (end 89.154 83.058) (width 0.5) (layer "B.Cu") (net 16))
 (segment (start 97.038 88.783) (end 90.307 88.783) (width 0.5) (layer "B.Cu") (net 16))
 (segment (start 91.821 79.502) (end 91.821 82.423) (width 0.5) (layer "B.Cu") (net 16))
 (segment (start 93.599 70.415) (end 91.51 70.415) (width 0.5) (layer "B.Cu") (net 16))
 (segment (start 90.307 88.783) (end 89.154 87.63) (width 0.5) (layer "B.Cu") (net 16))
 (segment (start 97.028 78.232) (end 97.038 78.242) (width 0.5) (layer "B.Cu") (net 17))
 (segment (start 97.038 78.242) (end 97.038 81.163) (width 0.5) (layer "B.Cu") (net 17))
 (segment (start 97.028 77.724) (end 97.028 78.232) (width 0.5) (layer "B.Cu") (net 17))
 (segment (start 93.599 74.295) (end 97.028 77.724) (width 0.5) (layer "B.Cu") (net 17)))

